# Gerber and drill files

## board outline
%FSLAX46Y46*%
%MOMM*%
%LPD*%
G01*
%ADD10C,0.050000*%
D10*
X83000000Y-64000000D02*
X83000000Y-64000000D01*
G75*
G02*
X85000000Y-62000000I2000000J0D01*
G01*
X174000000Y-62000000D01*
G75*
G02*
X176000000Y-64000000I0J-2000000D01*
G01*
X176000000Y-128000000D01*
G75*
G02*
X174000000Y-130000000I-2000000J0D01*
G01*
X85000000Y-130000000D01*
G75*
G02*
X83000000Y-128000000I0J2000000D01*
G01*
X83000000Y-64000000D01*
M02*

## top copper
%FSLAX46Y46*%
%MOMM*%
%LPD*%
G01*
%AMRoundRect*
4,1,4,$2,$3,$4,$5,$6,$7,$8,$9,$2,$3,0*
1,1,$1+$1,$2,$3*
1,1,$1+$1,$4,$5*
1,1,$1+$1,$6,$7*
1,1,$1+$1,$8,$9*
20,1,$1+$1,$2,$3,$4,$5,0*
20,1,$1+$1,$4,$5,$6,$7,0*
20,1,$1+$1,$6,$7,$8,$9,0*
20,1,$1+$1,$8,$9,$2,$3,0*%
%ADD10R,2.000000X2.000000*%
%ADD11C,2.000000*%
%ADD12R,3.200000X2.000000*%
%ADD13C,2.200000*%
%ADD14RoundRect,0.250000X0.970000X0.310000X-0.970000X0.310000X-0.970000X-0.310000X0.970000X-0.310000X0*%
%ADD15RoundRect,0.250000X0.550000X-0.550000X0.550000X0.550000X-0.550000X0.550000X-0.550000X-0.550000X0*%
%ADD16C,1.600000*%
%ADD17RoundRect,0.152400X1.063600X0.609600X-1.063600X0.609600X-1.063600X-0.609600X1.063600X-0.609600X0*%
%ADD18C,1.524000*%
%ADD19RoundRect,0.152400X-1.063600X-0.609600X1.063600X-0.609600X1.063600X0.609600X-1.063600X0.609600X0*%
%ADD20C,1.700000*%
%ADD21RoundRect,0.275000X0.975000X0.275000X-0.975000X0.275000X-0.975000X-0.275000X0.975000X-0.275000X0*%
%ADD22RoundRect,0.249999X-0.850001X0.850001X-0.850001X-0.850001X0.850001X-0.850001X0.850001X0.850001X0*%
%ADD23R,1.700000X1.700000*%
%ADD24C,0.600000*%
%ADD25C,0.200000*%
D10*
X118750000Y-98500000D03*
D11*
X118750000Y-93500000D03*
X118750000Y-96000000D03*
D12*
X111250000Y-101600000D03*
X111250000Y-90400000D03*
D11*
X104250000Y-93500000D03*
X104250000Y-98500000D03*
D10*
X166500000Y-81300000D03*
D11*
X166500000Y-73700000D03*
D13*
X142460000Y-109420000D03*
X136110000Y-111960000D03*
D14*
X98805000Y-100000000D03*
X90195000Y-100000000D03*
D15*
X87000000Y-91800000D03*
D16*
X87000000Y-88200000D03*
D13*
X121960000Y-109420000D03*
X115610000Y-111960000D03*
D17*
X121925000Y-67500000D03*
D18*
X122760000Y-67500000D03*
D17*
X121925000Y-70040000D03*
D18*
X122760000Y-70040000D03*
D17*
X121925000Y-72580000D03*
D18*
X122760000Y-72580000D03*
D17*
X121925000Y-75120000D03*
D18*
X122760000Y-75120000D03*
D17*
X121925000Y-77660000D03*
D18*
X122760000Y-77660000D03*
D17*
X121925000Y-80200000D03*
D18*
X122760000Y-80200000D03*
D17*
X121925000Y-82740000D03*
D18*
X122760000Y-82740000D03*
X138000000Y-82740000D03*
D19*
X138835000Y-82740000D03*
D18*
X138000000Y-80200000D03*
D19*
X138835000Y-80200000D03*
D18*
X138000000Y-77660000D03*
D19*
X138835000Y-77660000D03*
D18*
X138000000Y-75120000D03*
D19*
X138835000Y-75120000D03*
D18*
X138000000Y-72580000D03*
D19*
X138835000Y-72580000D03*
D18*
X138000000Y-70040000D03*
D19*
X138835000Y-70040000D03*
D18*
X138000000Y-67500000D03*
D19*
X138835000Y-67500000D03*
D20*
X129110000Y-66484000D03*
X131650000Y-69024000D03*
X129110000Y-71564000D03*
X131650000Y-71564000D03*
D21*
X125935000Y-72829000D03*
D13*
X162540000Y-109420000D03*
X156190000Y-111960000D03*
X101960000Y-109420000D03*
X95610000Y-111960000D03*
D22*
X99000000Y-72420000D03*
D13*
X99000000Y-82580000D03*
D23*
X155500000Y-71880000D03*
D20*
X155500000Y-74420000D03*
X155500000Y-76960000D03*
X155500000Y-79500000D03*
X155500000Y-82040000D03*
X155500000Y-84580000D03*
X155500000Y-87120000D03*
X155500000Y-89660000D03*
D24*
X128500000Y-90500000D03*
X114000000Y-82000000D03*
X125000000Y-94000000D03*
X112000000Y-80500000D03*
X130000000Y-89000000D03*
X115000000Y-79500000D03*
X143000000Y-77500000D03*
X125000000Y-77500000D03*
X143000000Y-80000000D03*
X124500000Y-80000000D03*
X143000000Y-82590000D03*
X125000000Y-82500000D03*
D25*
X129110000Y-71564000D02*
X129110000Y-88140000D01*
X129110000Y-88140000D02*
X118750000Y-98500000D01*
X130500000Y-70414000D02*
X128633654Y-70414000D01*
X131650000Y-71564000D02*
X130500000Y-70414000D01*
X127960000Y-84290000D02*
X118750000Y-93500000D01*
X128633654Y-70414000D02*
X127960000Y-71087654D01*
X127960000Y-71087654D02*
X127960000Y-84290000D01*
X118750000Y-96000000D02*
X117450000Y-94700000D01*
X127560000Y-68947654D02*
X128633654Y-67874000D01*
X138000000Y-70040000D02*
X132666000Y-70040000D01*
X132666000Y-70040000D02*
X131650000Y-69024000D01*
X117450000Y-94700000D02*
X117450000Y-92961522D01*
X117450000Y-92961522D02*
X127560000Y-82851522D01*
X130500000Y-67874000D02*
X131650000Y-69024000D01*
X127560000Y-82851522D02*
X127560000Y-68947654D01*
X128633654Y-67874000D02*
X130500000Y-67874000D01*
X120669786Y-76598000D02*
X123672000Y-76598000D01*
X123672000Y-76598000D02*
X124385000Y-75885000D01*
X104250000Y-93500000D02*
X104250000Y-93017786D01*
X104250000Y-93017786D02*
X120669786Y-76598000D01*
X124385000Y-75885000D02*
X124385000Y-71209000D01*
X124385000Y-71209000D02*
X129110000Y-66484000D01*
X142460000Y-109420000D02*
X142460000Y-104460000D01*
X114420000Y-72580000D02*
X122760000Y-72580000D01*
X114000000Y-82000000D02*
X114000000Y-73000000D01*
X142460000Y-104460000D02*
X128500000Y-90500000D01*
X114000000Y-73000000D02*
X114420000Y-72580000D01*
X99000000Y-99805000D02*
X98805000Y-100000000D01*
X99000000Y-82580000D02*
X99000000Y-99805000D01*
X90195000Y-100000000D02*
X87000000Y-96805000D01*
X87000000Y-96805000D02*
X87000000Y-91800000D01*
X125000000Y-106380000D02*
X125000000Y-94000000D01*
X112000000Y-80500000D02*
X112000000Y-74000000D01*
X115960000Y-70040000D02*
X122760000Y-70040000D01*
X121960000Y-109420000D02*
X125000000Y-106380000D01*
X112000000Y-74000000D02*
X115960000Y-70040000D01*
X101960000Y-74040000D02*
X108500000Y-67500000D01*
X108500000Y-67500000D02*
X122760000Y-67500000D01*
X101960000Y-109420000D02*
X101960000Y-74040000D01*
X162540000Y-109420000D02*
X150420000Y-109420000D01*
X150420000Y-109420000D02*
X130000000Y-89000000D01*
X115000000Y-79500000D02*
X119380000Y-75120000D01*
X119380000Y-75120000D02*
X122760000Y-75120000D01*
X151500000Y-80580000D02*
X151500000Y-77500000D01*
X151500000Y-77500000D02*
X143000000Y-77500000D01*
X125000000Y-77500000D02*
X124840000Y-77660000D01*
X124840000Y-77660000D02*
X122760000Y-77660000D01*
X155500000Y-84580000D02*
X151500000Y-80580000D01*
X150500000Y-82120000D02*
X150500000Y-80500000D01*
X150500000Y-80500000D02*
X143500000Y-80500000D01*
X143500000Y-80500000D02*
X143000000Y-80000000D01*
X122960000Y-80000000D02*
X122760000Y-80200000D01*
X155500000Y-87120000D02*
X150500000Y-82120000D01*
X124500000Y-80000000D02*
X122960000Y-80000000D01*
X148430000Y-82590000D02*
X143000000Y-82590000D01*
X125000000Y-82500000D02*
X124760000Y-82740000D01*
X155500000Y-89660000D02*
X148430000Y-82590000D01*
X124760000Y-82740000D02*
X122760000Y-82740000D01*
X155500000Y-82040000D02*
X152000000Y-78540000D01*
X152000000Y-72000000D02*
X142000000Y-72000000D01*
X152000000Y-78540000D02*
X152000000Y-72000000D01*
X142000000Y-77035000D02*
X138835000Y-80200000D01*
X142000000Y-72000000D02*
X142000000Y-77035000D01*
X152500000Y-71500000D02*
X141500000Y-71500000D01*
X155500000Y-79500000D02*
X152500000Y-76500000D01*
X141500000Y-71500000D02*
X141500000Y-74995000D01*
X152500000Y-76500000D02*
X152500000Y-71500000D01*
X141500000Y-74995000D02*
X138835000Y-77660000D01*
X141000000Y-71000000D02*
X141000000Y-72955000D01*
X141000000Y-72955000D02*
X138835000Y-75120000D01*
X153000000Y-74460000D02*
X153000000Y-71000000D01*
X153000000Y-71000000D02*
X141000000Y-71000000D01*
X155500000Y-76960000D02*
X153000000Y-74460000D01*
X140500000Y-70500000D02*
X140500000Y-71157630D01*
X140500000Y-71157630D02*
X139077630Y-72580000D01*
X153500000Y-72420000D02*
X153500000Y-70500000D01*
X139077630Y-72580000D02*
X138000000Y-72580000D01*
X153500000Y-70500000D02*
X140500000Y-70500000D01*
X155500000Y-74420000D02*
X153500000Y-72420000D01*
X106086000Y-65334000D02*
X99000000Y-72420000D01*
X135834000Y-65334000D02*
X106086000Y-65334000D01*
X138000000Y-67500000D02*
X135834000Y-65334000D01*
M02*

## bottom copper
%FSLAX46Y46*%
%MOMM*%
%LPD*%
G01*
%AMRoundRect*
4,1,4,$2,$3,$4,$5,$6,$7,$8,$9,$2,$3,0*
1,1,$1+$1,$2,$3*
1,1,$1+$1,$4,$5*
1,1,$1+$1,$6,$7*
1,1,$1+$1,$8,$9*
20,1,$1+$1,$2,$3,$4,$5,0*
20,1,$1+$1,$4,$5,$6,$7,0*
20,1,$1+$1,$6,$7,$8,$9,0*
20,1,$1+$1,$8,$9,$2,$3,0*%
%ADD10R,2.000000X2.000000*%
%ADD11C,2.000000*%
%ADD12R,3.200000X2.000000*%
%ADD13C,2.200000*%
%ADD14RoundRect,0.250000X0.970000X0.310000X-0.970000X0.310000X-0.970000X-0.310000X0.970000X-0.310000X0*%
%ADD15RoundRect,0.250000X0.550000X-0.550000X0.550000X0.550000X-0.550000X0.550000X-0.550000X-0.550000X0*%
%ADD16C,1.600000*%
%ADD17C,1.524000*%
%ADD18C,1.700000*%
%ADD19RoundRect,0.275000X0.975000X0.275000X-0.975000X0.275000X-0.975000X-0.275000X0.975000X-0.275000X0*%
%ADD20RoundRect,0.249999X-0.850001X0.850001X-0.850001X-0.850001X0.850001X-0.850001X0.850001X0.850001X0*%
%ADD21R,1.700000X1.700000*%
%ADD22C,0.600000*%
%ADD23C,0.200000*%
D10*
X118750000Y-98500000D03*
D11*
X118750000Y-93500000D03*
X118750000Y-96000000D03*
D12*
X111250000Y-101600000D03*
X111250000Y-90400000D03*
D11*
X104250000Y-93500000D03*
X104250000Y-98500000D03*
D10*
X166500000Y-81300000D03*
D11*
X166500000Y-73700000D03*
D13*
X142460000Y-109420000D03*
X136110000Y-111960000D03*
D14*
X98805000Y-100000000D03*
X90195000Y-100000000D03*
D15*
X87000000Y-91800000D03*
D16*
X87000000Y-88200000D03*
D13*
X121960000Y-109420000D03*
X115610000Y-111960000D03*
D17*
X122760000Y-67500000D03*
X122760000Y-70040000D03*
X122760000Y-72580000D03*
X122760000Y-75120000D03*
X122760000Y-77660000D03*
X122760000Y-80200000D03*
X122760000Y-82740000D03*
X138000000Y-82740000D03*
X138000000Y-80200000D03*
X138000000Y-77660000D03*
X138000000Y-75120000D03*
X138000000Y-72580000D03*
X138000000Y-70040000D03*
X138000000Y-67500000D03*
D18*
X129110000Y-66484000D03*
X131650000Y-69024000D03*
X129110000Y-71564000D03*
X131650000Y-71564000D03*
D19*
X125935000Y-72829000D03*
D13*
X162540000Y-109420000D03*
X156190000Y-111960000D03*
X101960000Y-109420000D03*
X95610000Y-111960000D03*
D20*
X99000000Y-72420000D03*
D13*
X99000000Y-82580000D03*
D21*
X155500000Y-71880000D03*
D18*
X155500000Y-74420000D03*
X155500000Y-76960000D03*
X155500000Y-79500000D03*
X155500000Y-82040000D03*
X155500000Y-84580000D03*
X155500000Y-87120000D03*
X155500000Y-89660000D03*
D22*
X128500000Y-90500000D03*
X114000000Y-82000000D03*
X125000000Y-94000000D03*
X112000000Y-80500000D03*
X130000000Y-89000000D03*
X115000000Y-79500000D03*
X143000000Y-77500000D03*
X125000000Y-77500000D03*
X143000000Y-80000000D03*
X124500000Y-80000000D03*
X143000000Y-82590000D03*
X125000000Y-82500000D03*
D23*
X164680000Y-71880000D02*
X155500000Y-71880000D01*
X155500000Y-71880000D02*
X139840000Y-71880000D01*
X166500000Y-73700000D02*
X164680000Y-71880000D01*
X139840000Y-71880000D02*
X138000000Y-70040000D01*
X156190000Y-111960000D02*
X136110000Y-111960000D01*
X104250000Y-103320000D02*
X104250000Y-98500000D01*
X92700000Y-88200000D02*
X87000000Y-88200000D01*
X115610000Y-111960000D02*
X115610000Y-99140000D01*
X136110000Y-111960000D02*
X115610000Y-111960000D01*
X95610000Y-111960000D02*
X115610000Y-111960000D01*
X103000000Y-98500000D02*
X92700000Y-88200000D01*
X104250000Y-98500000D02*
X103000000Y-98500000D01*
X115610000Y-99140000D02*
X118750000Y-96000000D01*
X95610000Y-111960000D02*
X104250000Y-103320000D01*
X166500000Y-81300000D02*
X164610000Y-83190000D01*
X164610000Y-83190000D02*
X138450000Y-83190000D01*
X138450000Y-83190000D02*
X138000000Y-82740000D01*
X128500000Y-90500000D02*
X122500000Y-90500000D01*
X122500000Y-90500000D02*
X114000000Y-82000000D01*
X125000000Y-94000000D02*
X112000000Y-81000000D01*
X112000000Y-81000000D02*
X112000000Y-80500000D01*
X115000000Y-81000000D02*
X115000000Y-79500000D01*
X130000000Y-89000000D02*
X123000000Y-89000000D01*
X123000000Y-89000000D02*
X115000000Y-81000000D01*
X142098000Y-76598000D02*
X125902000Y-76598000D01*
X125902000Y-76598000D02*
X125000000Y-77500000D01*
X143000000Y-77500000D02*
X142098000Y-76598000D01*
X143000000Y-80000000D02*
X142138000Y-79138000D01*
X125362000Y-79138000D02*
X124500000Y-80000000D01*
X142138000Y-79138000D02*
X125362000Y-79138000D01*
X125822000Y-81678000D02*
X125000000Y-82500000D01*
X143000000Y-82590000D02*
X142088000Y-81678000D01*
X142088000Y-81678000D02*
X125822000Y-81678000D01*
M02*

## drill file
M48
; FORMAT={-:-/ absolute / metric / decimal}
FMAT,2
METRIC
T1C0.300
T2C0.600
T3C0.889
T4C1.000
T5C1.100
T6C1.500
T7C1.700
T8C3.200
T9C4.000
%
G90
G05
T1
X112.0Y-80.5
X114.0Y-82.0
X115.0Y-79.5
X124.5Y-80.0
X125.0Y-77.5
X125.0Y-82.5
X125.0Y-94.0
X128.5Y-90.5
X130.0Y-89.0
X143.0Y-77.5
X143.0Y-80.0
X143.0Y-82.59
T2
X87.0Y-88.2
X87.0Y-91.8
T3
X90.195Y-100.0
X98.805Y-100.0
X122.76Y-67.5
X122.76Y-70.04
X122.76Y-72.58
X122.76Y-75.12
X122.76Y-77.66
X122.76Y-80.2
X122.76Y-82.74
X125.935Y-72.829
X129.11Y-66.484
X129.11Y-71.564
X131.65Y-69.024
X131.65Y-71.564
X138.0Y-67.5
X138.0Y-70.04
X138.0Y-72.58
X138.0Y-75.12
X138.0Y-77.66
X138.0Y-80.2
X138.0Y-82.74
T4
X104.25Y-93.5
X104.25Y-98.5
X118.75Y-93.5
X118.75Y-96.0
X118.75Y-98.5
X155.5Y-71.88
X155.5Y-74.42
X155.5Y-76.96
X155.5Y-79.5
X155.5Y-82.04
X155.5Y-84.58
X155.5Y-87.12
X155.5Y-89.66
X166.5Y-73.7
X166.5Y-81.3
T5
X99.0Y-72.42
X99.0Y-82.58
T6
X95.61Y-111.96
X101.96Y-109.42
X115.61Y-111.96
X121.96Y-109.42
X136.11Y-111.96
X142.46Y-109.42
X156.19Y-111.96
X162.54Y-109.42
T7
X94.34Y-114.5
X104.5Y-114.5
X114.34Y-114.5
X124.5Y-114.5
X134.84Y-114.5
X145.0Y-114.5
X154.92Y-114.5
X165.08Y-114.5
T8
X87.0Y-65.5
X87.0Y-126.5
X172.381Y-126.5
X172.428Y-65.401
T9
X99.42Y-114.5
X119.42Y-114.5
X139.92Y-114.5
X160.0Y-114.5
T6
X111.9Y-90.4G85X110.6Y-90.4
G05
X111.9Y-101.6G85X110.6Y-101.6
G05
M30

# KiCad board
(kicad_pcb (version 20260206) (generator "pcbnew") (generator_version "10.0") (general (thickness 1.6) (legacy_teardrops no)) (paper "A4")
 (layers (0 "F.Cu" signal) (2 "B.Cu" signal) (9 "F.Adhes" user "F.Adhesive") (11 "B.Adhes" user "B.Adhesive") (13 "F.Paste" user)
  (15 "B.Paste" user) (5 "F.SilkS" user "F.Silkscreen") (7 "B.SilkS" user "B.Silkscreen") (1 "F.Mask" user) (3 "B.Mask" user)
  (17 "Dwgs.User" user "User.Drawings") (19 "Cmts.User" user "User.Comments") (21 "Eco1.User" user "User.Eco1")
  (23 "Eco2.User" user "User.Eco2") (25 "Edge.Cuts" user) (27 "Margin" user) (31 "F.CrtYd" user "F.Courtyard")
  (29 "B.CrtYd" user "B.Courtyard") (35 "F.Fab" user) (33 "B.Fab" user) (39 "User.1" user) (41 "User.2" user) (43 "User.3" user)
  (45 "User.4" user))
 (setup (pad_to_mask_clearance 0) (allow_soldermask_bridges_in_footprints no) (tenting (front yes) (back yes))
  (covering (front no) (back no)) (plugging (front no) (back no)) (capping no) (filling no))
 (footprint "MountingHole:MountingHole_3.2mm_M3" (layer "F.Cu") (at 172.380609 126.5)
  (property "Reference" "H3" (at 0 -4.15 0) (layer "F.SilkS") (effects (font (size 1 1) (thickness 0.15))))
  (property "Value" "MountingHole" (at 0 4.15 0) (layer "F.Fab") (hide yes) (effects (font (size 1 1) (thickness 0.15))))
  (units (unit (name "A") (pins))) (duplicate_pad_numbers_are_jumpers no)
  (pad "" np_thru_hole circle (at 0 0) (size 3.2 3.2) (drill 3.2) (layers "*.Cu" "*.Mask")))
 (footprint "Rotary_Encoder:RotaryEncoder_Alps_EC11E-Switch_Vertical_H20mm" (layer "F.Cu") (at 118.75 98.5 180)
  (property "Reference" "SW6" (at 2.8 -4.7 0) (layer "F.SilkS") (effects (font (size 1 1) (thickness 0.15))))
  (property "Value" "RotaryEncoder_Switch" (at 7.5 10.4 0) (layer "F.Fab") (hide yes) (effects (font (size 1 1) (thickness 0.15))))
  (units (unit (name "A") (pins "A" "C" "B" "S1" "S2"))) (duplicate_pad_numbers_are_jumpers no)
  (pad "A" thru_hole rect (at 0 0 180) (size 2 2) (drill 1) (layers "*.Cu" "*.Mask") (remove_unused_layers no)
   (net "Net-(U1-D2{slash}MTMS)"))
  (pad "B" thru_hole circle (at 0 5 180) (size 2 2) (drill 1) (layers "*.Cu" "*.Mask") (remove_unused_layers no)
   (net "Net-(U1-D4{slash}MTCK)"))
  (pad "C" thru_hole circle (at 0 2.5 180) (size 2 2) (drill 1) (layers "*.Cu" "*.Mask") (remove_unused_layers no) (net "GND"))
  (pad "MP" thru_hole rect (at 7.5 -3.1 180) (size 3.2 2) (drill oval 2.8 1.5) (layers "*.Cu" "*.Mask") (remove_unused_layers no))
  (pad "MP" thru_hole rect (at 7.5 8.1 180) (size 3.2 2) (drill oval 2.8 1.5) (layers "*.Cu" "*.Mask") (remove_unused_layers no))
  (pad "S1" thru_hole circle (at 14.5 5 180) (size 2 2) (drill 1) (layers "*.Cu" "*.Mask") (remove_unused_layers no)
   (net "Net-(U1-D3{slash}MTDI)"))
  (pad "S2" thru_hole circle (at 14.5 0 180) (size 2 2) (drill 1) (layers "*.Cu" "*.Mask") (remove_unused_layers no) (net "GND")))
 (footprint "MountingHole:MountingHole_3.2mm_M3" (layer "F.Cu") (at 172.4285 65.401372)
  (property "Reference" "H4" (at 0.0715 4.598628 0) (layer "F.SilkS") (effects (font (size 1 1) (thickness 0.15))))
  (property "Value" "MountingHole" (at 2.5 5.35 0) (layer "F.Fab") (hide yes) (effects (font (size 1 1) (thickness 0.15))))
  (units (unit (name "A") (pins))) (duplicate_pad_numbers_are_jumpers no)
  (pad "" np_thru_hole circle (at 0 0) (size 3.2 3.2) (drill 3.2) (layers "*.Cu" "*.Mask")))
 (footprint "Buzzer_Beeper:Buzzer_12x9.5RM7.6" (layer "F.Cu") (at 166.5 81.3 90)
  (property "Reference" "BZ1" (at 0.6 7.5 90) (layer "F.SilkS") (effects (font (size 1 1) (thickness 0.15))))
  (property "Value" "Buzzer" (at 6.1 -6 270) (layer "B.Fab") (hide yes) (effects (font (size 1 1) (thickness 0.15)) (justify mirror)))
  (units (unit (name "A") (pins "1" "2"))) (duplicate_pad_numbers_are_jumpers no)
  (pad "1" thru_hole rect (at 0 0 90) (size 2 2) (drill 1) (layers "*.Cu" "*.Mask") (remove_unused_layers no) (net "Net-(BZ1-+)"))
  (pad "2" thru_hole circle (at 7.6 0 90) (size 2 2) (drill 1) (layers "*.Cu" "*.Mask") (remove_unused_layers no) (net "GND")))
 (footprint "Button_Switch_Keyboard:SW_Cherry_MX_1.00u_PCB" (layer "F.Cu") (at 142.46 109.42)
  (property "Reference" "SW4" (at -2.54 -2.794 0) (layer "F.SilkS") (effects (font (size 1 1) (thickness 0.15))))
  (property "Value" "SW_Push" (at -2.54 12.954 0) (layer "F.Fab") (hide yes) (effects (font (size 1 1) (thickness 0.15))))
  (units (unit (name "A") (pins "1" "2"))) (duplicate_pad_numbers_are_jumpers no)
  (pad "" np_thru_hole circle (at -7.62 5.08) (size 1.7 1.7) (drill 1.7) (layers "*.Cu" "*.Mask"))
  (pad "" np_thru_hole circle (at -2.54 5.08) (size 4 4) (drill 4) (layers "*.Cu" "*.Mask"))
  (pad "" np_thru_hole circle (at 2.54 5.08) (size 1.7 1.7) (drill 1.7) (layers "*.Cu" "*.Mask"))
  (pad "1" thru_hole circle (at 0 0) (size 2.2 2.2) (drill 1.5) (layers "*.Cu" "*.Mask") (remove_unused_layers no) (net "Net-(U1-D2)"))
  (pad "2" thru_hole circle (at -6.35 2.54) (size 2.2 2.2) (drill 1.5) (layers "*.Cu" "*.Mask") (remove_unused_layers no) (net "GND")))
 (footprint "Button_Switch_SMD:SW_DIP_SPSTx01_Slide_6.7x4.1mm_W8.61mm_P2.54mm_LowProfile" (layer "F.Cu") (at 94.5 100 180)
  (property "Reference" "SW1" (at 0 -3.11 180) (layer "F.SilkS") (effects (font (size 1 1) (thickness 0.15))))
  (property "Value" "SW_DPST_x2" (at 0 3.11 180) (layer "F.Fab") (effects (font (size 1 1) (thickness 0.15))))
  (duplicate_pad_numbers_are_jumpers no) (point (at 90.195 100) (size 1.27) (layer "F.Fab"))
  (pad "1" thru_hole roundrect (at -4.305 0 180) (size 2.44 1.12) (drill 0.889) (layers "*.Cu" "*.Mask" "F.Paste") (remove_unused_layers no)
   (roundrect_rratio 0.223214) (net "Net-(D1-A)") (zone_connect 2))
  (pad "2" thru_hole roundrect (at 4.305 0 180) (size 2.44 1.12) (drill 0.889) (layers "*.Cu" "*.Mask") (remove_unused_layers no)
   (roundrect_rratio 0.223214) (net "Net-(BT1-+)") (zone_connect 2)))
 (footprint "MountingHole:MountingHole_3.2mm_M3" (layer "F.Cu") (at 87 126.5)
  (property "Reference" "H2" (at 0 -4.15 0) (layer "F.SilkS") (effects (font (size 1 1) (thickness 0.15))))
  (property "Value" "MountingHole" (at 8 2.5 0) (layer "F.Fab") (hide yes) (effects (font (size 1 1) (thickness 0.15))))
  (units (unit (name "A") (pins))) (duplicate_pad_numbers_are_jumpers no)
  (pad "" np_thru_hole circle (at 0 0) (size 3.2 3.2) (drill 3.2) (layers "*.Cu" "*.Mask")))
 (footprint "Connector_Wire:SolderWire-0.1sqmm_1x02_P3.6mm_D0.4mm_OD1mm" (layer "F.Cu") (at 87 91.8 90)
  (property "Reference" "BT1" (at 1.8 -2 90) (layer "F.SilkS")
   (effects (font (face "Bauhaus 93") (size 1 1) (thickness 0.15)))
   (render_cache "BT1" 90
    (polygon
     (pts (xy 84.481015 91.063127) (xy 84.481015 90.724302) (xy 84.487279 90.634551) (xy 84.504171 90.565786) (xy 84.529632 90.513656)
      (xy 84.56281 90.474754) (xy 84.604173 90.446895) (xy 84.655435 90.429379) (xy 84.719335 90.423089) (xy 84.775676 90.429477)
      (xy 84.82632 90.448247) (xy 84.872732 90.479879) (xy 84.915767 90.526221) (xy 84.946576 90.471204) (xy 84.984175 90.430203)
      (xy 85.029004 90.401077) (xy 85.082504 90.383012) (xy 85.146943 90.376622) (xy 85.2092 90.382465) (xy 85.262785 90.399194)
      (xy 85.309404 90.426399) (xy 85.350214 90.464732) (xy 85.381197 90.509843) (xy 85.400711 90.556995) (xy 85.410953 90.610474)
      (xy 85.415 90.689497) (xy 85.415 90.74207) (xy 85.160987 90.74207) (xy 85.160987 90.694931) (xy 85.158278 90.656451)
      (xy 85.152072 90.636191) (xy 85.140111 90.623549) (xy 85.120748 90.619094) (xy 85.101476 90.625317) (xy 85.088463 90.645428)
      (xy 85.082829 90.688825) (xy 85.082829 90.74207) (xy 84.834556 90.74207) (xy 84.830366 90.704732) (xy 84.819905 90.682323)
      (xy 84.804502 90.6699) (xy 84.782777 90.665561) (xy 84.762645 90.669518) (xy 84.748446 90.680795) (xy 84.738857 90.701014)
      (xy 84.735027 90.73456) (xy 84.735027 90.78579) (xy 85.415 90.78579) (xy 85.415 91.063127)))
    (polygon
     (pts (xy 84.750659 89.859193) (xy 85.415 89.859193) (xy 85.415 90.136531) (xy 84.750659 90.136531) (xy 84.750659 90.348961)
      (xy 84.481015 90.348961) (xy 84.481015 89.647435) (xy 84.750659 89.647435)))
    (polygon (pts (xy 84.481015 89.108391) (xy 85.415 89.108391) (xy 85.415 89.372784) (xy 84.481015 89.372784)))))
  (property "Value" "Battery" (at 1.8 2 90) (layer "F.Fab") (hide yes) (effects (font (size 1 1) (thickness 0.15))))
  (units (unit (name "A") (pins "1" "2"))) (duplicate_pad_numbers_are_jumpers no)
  (pad "1" thru_hole roundrect (at 0 0 90) (size 1.6 1.6) (drill 0.6) (layers "*.Cu" "*.Mask") (remove_unused_layers no)
   (roundrect_rratio 0.15625) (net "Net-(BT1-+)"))
  (pad "2" thru_hole circle (at 3.6 0 90) (size 1.6 1.6) (drill 0.6) (layers "*.Cu" "*.Mask") (remove_unused_layers no) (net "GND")))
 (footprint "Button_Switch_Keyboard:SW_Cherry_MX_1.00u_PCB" (layer "F.Cu") (at 121.96 109.42)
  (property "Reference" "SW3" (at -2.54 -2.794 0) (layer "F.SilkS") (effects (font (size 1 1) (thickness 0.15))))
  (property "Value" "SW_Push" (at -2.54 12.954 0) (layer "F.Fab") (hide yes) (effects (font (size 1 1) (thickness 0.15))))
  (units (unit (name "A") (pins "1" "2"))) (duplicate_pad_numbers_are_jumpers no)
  (pad "" np_thru_hole circle (at -7.62 5.08) (size 1.7 1.7) (drill 1.7) (layers "*.Cu" "*.Mask"))
  (pad "" np_thru_hole circle (at -2.54 5.08) (size 4 4) (drill 4) (layers "*.Cu" "*.Mask"))
  (pad "" np_thru_hole circle (at 2.54 5.08) (size 1.7 1.7) (drill 1.7) (layers "*.Cu" "*.Mask"))
  (pad "1" thru_hole circle (at 0 0) (size 2.2 2.2) (drill 1.5) (layers "*.Cu" "*.Mask") (remove_unused_layers no) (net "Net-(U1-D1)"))
  (pad "2" thru_hole circle (at -6.35 2.54) (size 2.2 2.2) (drill 1.5) (layers "*.Cu" "*.Mask") (remove_unused_layers no) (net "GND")))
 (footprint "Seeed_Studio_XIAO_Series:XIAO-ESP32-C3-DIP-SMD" (layer "F.Cu") (at 130.38 75.12 90)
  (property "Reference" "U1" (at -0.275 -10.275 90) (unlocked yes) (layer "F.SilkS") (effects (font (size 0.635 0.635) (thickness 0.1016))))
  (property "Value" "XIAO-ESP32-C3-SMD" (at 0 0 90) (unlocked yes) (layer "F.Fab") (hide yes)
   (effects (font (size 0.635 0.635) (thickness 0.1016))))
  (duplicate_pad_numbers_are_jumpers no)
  (pad "1" smd roundrect (at 7.62 -8.455 180) (size 2.432 1.524) (layers "F.Cu" "F.Mask") (roundrect_rratio 0.1) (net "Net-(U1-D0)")
   (thermal_bridge_angle 45))
  (pad "1" thru_hole circle (at 7.62 -7.62 180) (size 1.524 1.524) (drill 0.889) (layers "*.Cu" "*.Mask") (remove_unused_layers no)
   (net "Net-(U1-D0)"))
  (pad "2" smd roundrect (at 5.08 -8.455 180) (size 2.432 1.524) (layers "F.Cu" "F.Mask") (roundrect_rratio 0.1) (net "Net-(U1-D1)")
   (thermal_bridge_angle 45))
  (pad "2" thru_hole circle (at 5.08 -7.62 180) (size 1.524 1.524) (drill 0.889) (layers "*.Cu" "*.Mask") (remove_unused_layers no)
   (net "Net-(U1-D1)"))
  (pad "3" smd roundrect (at 2.54 -8.455 180) (size 2.432 1.524) (layers "F.Cu" "F.Mask") (roundrect_rratio 0.1) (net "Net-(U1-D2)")
   (thermal_bridge_angle 45))
  (pad "3" thru_hole circle (at 2.54 -7.62 180) (size 1.524 1.524) (drill 0.889) (layers "*.Cu" "*.Mask") (remove_unused_layers no)
   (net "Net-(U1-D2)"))
  (pad "4" smd roundrect (at 0 -8.455 180) (size 2.432 1.524) (layers "F.Cu" "F.Mask") (roundrect_rratio 0.1) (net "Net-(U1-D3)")
   (thermal_bridge_angle 45))
  (pad "4" thru_hole circle (at 0 -7.62 180) (size 1.524 1.524) (drill 0.889) (layers "*.Cu" "*.Mask") (remove_unused_layers no)
   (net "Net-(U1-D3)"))
  (pad "5" smd roundrect (at -2.54 -8.455 180) (size 2.432 1.524) (layers "F.Cu" "F.Mask") (roundrect_rratio 0.1) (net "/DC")
   (thermal_bridge_angle 45))
  (pad "5" thru_hole circle (at -2.54 -7.62 180) (size 1.524 1.524) (drill 0.889) (layers "*.Cu" "*.Mask") (remove_unused_layers no)
   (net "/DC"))
  (pad "6" smd roundrect (at -5.08 -8.455 180) (size 2.432 1.524) (layers "F.Cu" "F.Mask") (roundrect_rratio 0.1) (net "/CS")
   (thermal_bridge_angle 45))
  (pad "6" thru_hole circle (at -5.08 -7.62 180) (size 1.524 1.524) (drill 0.889) (layers "*.Cu" "*.Mask") (remove_unused_layers no)
   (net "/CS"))
  (pad "7" smd roundrect (at -7.62 -8.455 180) (size 2.432 1.524) (layers "F.Cu" "F.Mask") (roundrect_rratio 0.1) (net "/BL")
   (thermal_bridge_angle 45))
  (pad "7" thru_hole circle (at -7.62 -7.62 180) (size 1.524 1.524) (drill 0.889) (layers "*.Cu" "*.Mask") (remove_unused_layers no)
   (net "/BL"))
  (pad "8" thru_hole circle (at -7.62 7.62) (size 1.524 1.524) (drill 0.889) (layers "*.Cu" "*.Mask") (remove_unused_layers no)
   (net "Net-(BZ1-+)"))
  (pad "8" smd roundrect (at -7.62 8.455) (size 2.432 1.524) (layers "F.Cu" "F.Mask") (roundrect_rratio 0.1) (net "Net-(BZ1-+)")
   (thermal_bridge_angle 45))
  (pad "9" thru_hole circle (at -5.08 7.62) (size 1.524 1.524) (drill 0.889) (layers "*.Cu" "*.Mask") (remove_unused_layers no) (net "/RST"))
  (pad "9" smd roundrect (at -5.08 8.455) (size 2.432 1.524) (layers "F.Cu" "F.Mask") (roundrect_rratio 0.1) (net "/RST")
   (thermal_bridge_angle 45))
  (pad "10" thru_hole circle (at -2.54 7.62) (size 1.524 1.524) (drill 0.889) (layers "*.Cu" "*.Mask") (remove_unused_layers no)
   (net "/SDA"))
  (pad "10" smd roundrect (at -2.54 8.455) (size 2.432 1.524) (layers "F.Cu" "F.Mask") (roundrect_rratio 0.1) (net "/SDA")
   (thermal_bridge_angle 45))
  (pad "11" thru_hole circle (at 0 7.62) (size 1.524 1.524) (drill 0.889) (layers "*.Cu" "*.Mask") (remove_unused_layers no) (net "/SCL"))
  (pad "11" smd roundrect (at 0 8.455) (size 2.432 1.524) (layers "F.Cu" "F.Mask") (roundrect_rratio 0.1) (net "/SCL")
   (thermal_bridge_angle 45))
  (pad "12" thru_hole circle (at 2.54 7.62) (size 1.524 1.524) (drill 0.889) (layers "*.Cu" "*.Mask") (remove_unused_layers no)
   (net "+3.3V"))
  (pad "12" smd roundrect (at 2.54 8.455) (size 2.432 1.524) (layers "F.Cu" "F.Mask") (roundrect_rratio 0.1) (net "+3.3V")
   (thermal_bridge_angle 45))
  (pad "13" thru_hole circle (at 5.08 7.62) (size 1.524 1.524) (drill 0.889) (layers "*.Cu" "*.Mask") (remove_unused_layers no) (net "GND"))
  (pad "13" smd roundrect (at 5.08 8.455) (size 2.432 1.524) (layers "F.Cu" "F.Mask") (roundrect_rratio 0.1) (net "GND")
   (thermal_bridge_angle 45))
  (pad "14" thru_hole circle (at 7.62 7.62) (size 1.524 1.524) (drill 0.889) (layers "*.Cu" "*.Mask") (remove_unused_layers no)
   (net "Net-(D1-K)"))
  (pad "14" smd roundrect (at 7.62 8.455) (size 2.432 1.524) (layers "F.Cu" "F.Mask") (roundrect_rratio 0.1) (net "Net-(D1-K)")
   (thermal_bridge_angle 45))
  (pad "15" thru_hole circle (at 8.636 -1.27) (size 1.7 1.7) (drill 0.889) (layers "*.Cu" "*.Mask") (remove_unused_layers no)
   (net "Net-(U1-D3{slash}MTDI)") (zone_connect 2))
  (pad "18" thru_hole circle (at 6.096 1.27) (size 1.7 1.7) (drill 0.889) (layers "*.Cu" "*.Mask") (remove_unused_layers no) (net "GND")
   (zone_connect 2))
  (pad "19" thru_hole circle (at 3.556 -1.27) (size 1.7 1.7) (drill 0.889) (layers "*.Cu" "*.Mask") (remove_unused_layers no)
   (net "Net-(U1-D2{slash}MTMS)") (zone_connect 2))
  (pad "20" thru_hole circle (at 3.556 1.27) (size 1.7 1.7) (drill 0.889) (layers "*.Cu" "F.Mask") (remove_unused_layers no)
   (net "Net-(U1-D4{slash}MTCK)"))
  (pad "GND" thru_hole roundrect (at 2.291 -4.445 180) (size 2.5 1.1) (drill 0.889) (layers "*.Cu" "*.Mask") (remove_unused_layers no)
   (roundrect_rratio 0.25) (die_length 2) (thermal_bridge_angle 45)))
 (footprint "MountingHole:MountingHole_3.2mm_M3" (layer "F.Cu") (at 87 65.5)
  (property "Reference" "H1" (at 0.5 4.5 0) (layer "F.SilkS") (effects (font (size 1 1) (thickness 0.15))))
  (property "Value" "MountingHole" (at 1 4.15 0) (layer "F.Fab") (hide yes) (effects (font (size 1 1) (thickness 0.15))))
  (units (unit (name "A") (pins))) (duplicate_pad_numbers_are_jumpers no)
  (pad "" np_thru_hole circle (at 0 0) (size 3.2 3.2) (drill 3.2) (layers "*.Cu" "*.Mask")))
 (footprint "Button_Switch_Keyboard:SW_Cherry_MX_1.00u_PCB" (layer "F.Cu") (at 162.54 109.42)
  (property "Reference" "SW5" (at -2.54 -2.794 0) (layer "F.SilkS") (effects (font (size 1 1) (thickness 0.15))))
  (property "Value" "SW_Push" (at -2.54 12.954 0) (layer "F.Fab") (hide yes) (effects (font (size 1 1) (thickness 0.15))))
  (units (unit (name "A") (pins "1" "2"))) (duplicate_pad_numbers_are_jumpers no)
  (pad "" np_thru_hole circle (at -7.62 5.08) (size 1.7 1.7) (drill 1.7) (layers "*.Cu" "*.Mask"))
  (pad "" np_thru_hole circle (at -2.54 5.08) (size 4 4) (drill 4) (layers "*.Cu" "*.Mask"))
  (pad "" np_thru_hole circle (at 2.54 5.08) (size 1.7 1.7) (drill 1.7) (layers "*.Cu" "*.Mask"))
  (pad "1" thru_hole circle (at 0 0) (size 2.2 2.2) (drill 1.5) (layers "*.Cu" "*.Mask") (remove_unused_layers no) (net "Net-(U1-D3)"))
  (pad "2" thru_hole circle (at -6.35 2.54) (size 2.2 2.2) (drill 1.5) (layers "*.Cu" "*.Mask") (remove_unused_layers no) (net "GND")))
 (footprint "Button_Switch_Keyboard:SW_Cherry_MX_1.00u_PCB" (layer "F.Cu") (at 101.96 109.42)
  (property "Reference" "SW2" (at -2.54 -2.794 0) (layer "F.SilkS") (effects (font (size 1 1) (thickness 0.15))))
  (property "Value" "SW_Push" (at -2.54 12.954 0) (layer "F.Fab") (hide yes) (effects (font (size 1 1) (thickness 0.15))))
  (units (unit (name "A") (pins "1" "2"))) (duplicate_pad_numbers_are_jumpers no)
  (pad "" np_thru_hole circle (at -7.62 5.08) (size 1.7 1.7) (drill 1.7) (layers "*.Cu" "*.Mask"))
  (pad "" np_thru_hole circle (at -2.54 5.08) (size 4 4) (drill 4) (layers "*.Cu" "*.Mask"))
  (pad "" np_thru_hole circle (at 2.54 5.08) (size 1.7 1.7) (drill 1.7) (layers "*.Cu" "*.Mask"))
  (pad "1" thru_hole circle (at 0 0) (size 2.2 2.2) (drill 1.5) (layers "*.Cu" "*.Mask") (remove_unused_layers no) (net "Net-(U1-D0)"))
  (pad "2" thru_hole circle (at -6.35 2.54) (size 2.2 2.2) (drill 1.5) (layers "*.Cu" "*.Mask") (remove_unused_layers no) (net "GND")))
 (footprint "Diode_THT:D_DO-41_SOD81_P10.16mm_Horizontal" (layer "B.Cu") (at 99 72.42 -90)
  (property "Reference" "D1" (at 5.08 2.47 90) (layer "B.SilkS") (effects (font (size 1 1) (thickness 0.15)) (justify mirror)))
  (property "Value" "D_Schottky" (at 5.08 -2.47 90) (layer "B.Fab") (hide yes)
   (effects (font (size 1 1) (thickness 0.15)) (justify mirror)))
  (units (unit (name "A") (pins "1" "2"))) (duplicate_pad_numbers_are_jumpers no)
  (pad "1" thru_hole roundrect (at 0 0 270) (size 2.2 2.2) (drill 1.1) (layers "*.Cu" "*.Mask") (remove_unused_layers no)
   (roundrect_rratio 0.113636) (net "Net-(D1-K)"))
  (pad "2" thru_hole circle (at 10.16 0 270) (size 2.2 2.2) (drill 1.1) (layers "*.Cu" "*.Mask") (remove_unused_layers no)
   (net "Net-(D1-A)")))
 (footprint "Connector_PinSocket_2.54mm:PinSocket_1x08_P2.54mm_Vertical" (layer "B.Cu") (at 155.5 71.88 180)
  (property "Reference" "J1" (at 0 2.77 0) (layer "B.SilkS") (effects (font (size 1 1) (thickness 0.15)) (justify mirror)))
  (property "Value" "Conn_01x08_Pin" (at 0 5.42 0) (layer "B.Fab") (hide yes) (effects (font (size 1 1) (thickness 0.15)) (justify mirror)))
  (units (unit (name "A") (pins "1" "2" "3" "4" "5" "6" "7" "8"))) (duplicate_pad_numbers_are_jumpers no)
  (pad "1" thru_hole rect (at 0 0 180) (size 1.7 1.7) (drill 1) (layers "*.Cu" "*.Mask") (remove_unused_layers no) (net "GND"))
  (pad "2" thru_hole circle (at 0 -2.54 180) (size 1.7 1.7) (drill 1) (layers "*.Cu" "*.Mask") (remove_unused_layers no) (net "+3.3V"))
  (pad "3" thru_hole circle (at 0 -5.08 180) (size 1.7 1.7) (drill 1) (layers "*.Cu" "*.Mask") (remove_unused_layers no) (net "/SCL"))
  (pad "4" thru_hole circle (at 0 -7.62 180) (size 1.7 1.7) (drill 1) (layers "*.Cu" "*.Mask") (remove_unused_layers no) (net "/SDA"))
  (pad "5" thru_hole circle (at 0 -10.16 180) (size 1.7 1.7) (drill 1) (layers "*.Cu" "*.Mask") (remove_unused_layers no) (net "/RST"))
  (pad "6" thru_hole circle (at 0 -12.7 180) (size 1.7 1.7) (drill 1) (layers "*.Cu" "*.Mask") (remove_unused_layers no) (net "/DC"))
  (pad "7" thru_hole circle (at 0 -15.24 180) (size 1.7 1.7) (drill 1) (layers "*.Cu" "*.Mask") (remove_unused_layers no) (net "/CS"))
  (pad "8" thru_hole circle (at 0 -17.78 180) (size 1.7 1.7) (drill 1) (layers "*.Cu" "*.Mask") (remove_unused_layers no) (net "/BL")))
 (gr_rect (start 83 62) (end 176 130) (radius 2) (stroke (width 0.05) (type solid)) (fill no) (layer "Edge.Cuts"))
 (segment (start 129.11 71.564) (end 129.11 88.14) (width 0.2) (layer "F.Cu") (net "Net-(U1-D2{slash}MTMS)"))
 (segment (start 129.11 88.14) (end 118.75 98.5) (width 0.2) (layer "F.Cu") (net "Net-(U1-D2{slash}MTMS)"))
 (segment (start 130.5 70.414) (end 128.633654 70.414) (width 0.2) (layer "F.Cu") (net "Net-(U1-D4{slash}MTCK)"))
 (segment (start 131.65 71.564) (end 130.5 70.414) (width 0.2) (layer "F.Cu") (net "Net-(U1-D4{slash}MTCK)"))
 (segment (start 127.96 84.29) (end 118.75 93.5) (width 0.2) (layer "F.Cu") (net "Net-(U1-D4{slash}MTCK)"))
 (segment (start 128.633654 70.414) (end 127.96 71.087654) (width 0.2) (layer "F.Cu") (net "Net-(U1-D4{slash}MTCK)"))
 (segment (start 127.96 71.087654) (end 127.96 84.29) (width 0.2) (layer "F.Cu") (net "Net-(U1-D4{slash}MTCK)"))
 (segment (start 118.75 96) (end 117.45 94.7) (width 0.2) (layer "F.Cu") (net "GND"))
 (segment (start 127.56 68.947654) (end 128.633654 67.874) (width 0.2) (layer "F.Cu") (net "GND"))
 (segment (start 138 70.04) (end 132.666 70.04) (width 0.2) (layer "F.Cu") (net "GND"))
 (segment (start 132.666 70.04) (end 131.65 69.024) (width 0.2) (layer "F.Cu") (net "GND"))
 (segment (start 117.45 94.7) (end 117.45 92.961522) (width 0.2) (layer "F.Cu") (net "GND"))
 (segment (start 117.45 92.961522) (end 127.56 82.851522) (width 0.2) (layer "F.Cu") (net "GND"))
 (segment (start 130.5 67.874) (end 131.65 69.024) (width 0.2) (layer "F.Cu") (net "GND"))
 (segment (start 127.56 82.851522) (end 127.56 68.947654) (width 0.2) (layer "F.Cu") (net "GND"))
 (segment (start 128.633654 67.874) (end 130.5 67.874) (width 0.2) (layer "F.Cu") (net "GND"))
 (segment (start 164.68 71.88) (end 155.5 71.88) (width 0.2) (layer "B.Cu") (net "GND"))
 (segment (start 155.5 71.88) (end 139.84 71.88) (width 0.2) (layer "B.Cu") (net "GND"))
 (segment (start 166.5 73.7) (end 164.68 71.88) (width 0.2) (layer "B.Cu") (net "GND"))
 (segment (start 139.84 71.88) (end 138 70.04) (width 0.2) (layer "B.Cu") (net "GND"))
 (segment (start 156.19 111.96) (end 136.11 111.96) (width 0.2) (layer "B.Cu") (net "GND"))
 (segment (start 104.25 103.32) (end 104.25 98.5) (width 0.2) (layer "B.Cu") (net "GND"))
 (segment (start 92.7 88.2) (end 87 88.2) (width 0.2) (layer "B.Cu") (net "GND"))
 (segment (start 115.61 111.96) (end 115.61 99.14) (width 0.2) (layer "B.Cu") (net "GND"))
 (segment (start 136.11 111.96) (end 115.61 111.96) (width 0.2) (layer "B.Cu") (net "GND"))
 (segment (start 95.61 111.96) (end 115.61 111.96) (width 0.2) (layer "B.Cu") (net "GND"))
 (segment (start 103 98.5) (end 92.7 88.2) (width 0.2) (layer "B.Cu") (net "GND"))
 (segment (start 104.25 98.5) (end 103 98.5) (width 0.2) (layer "B.Cu") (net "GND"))
 (segment (start 115.61 99.14) (end 118.75 96) (width 0.2) (layer "B.Cu") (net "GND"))
 (segment (start 95.61 111.96) (end 104.25 103.32) (width 0.2) (layer "B.Cu") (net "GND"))
 (segment (start 120.669786 76.598) (end 123.672 76.598) (width 0.2) (layer "F.Cu") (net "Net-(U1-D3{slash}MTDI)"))
 (segment (start 123.672 76.598) (end 124.385 75.885) (width 0.2) (layer "F.Cu") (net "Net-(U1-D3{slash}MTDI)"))
 (segment (start 104.25 93.5) (end 104.25 93.017786) (width 0.2) (layer "F.Cu") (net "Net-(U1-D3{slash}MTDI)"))
 (segment (start 104.25 93.017786) (end 120.669786 76.598) (width 0.2) (layer "F.Cu") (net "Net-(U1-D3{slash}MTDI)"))
 (segment (start 124.385 75.885) (end 124.385 71.209) (width 0.2) (layer "F.Cu") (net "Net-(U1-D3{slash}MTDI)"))
 (segment (start 124.385 71.209) (end 129.11 66.484) (width 0.2) (layer "F.Cu") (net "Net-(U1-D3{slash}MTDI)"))
 (segment (start 166.5 81.3) (end 164.61 83.19) (width 0.2) (layer "B.Cu") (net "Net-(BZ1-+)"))
 (segment (start 164.61 83.19) (end 138.45 83.19) (width 0.2) (layer "B.Cu") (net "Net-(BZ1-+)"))
 (segment (start 138.45 83.19) (end 138 82.74) (width 0.2) (layer "B.Cu") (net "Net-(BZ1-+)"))
 (segment (start 142.46 109.42) (end 142.46 104.46) (width 0.2) (layer "F.Cu") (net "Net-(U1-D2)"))
 (segment (start 114.42 72.58) (end 122.76 72.58) (width 0.2) (layer "F.Cu") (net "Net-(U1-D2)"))
 (segment (start 114 82) (end 114 73) (width 0.2) (layer "F.Cu") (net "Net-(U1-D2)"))
 (segment (start 142.46 104.46) (end 128.5 90.5) (width 0.2) (layer "F.Cu") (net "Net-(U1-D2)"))
 (segment (start 114 73) (end 114.42 72.58) (width 0.2) (layer "F.Cu") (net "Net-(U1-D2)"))
 (via (at 128.5 90.5) (size 0.6) (drill 0.3) (layers "F.Cu" "B.Cu") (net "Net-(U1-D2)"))
 (via (at 114 82) (size 0.6) (drill 0.3) (layers "F.Cu" "B.Cu") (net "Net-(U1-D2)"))
 (segment (start 128.5 90.5) (end 122.5 90.5) (width 0.2) (layer "B.Cu") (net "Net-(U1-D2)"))
 (segment (start 122.5 90.5) (end 114 82) (width 0.2) (layer "B.Cu") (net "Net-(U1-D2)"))
 (segment (start 99 99.805) (end 98.805 100) (width 0.2) (layer "F.Cu") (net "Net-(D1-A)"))
 (segment (start 99 82.58) (end 99 99.805) (width 0.2) (layer "F.Cu") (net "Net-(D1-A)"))
 (segment (start 90.195 100) (end 87 96.805) (width 0.2) (layer "F.Cu") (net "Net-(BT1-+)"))
 (segment (start 87 96.805) (end 87 91.8) (width 0.2) (layer "F.Cu") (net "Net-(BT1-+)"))
 (segment (start 125 106.38) (end 125 94) (width 0.2) (layer "F.Cu") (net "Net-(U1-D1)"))
 (segment (start 112 80.5) (end 112 74) (width 0.2) (layer "F.Cu") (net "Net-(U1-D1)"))
 (segment (start 115.96 70.04) (end 122.76 70.04) (width 0.2) (layer "F.Cu") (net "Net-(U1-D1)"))
 (segment (start 121.96 109.42) (end 125 106.38) (width 0.2) (layer "F.Cu") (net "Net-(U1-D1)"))
 (segment (start 112 74) (end 115.96 70.04) (width 0.2) (layer "F.Cu") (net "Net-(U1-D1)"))
 (via (at 125 94) (size 0.6) (drill 0.3) (layers "F.Cu" "B.Cu") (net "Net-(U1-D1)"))
 (via (at 112 80.5) (size 0.6) (drill 0.3) (layers "F.Cu" "B.Cu") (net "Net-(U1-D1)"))
 (segment (start 125 94) (end 112 81) (width 0.2) (layer "B.Cu") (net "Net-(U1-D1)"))
 (segment (start 112 81) (end 112 80.5) (width 0.2) (layer "B.Cu") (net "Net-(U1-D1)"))
 (segment (start 101.96 74.04) (end 108.5 67.5) (width 0.2) (layer "F.Cu") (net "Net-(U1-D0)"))
 (segment (start 108.5 67.5) (end 122.76 67.5) (width 0.2) (layer "F.Cu") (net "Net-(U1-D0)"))
 (segment (start 101.96 109.42) (end 101.96 74.04) (width 0.2) (layer "F.Cu") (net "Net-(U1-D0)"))
 (segment (start 162.54 109.42) (end 150.42 109.42) (width 0.2) (layer "F.Cu") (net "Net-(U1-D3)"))
 (segment (start 150.42 109.42) (end 130 89) (width 0.2) (layer "F.Cu") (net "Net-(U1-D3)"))
 (segment (start 115 79.5) (end 119.38 75.12) (width 0.2) (layer "F.Cu") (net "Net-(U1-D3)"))
 (segment (start 119.38 75.12) (end 122.76 75.12) (width 0.2) (layer "F.Cu") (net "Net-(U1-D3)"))
 (via (at 130 89) (size 0.6) (drill 0.3) (layers "F.Cu" "B.Cu") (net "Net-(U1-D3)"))
 (via (at 115 79.5) (size 0.6) (drill 0.3) (layers "F.Cu" "B.Cu") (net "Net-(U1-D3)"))
 (segment (start 115 81) (end 115 79.5) (width 0.2) (layer "B.Cu") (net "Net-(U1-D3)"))
 (segment (start 130 89) (end 123 89) (width 0.2) (layer "B.Cu") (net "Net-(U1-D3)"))
 (segment (start 123 89) (end 115 81) (width 0.2) (layer "B.Cu") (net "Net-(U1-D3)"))
 (segment (start 151.5 80.58) (end 151.5 77.5) (width 0.2) (layer "F.Cu") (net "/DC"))
 (segment (start 151.5 77.5) (end 143 77.5) (width 0.2) (layer "F.Cu") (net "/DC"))
 (segment (start 125 77.5) (end 124.84 77.66) (width 0.2) (layer "F.Cu") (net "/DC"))
 (segment (start 124.84 77.66) (end 122.76 77.66) (width 0.2) (layer "F.Cu") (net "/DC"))
 (segment (start 155.5 84.58) (end 151.5 80.58) (width 0.2) (layer "F.Cu") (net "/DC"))
 (via (at 143 77.5) (size 0.6) (drill 0.3) (layers "F.Cu" "B.Cu") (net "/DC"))
 (via (at 125 77.5) (size 0.6) (drill 0.3) (layers "F.Cu" "B.Cu") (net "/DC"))
 (segment (start 142.098 76.598) (end 125.902 76.598) (width 0.2) (layer "B.Cu") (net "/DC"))
 (segment (start 125.902 76.598) (end 125 77.5) (width 0.2) (layer "B.Cu") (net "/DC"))
 (segment (start 143 77.5) (end 142.098 76.598) (width 0.2) (layer "B.Cu") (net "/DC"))
 (segment (start 150.5 82.12) (end 150.5 80.5) (width 0.2) (layer "F.Cu") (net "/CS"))
 (segment (start 150.5 80.5) (end 143.5 80.5) (width 0.2) (layer "F.Cu") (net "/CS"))
 (segment (start 143.5 80.5) (end 143 80) (width 0.2) (layer "F.Cu") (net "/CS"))
 (segment (start 122.96 80) (end 122.76 80.2) (width 0.2) (layer "F.Cu") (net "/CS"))
 (segment (start 155.5 87.12) (end 150.5 82.12) (width 0.2) (layer "F.Cu") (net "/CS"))
 (segment (start 124.5 80) (end 122.96 80) (width 0.2) (layer "F.Cu") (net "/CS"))
 (via (at 143 80) (size 0.6) (drill 0.3) (layers "F.Cu" "B.Cu") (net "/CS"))
 (via (at 124.5 80) (size 0.6) (drill 0.3) (layers "F.Cu" "B.Cu") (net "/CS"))
 (segment (start 143 80) (end 142.138 79.138) (width 0.2) (layer "B.Cu") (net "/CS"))
 (segment (start 125.362 79.138) (end 124.5 80) (width 0.2) (layer "B.Cu") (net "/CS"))
 (segment (start 142.138 79.138) (end 125.362 79.138) (width 0.2) (layer "B.Cu") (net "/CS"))
 (segment (start 148.43 82.59) (end 143 82.59) (width 0.2) (layer "F.Cu") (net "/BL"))
 (segment (start 125 82.5) (end 124.76 82.74) (width 0.2) (layer "F.Cu") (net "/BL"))
 (segment (start 155.5 89.66) (end 148.43 82.59) (width 0.2) (layer "F.Cu") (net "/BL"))
 (segment (start 124.76 82.74) (end 122.76 82.74) (width 0.2) (layer "F.Cu") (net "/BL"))
 (via (at 143 82.59) (size 0.6) (drill 0.3) (layers "F.Cu" "B.Cu") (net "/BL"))
 (via (at 125 82.5) (size 0.6) (drill 0.3) (layers "F.Cu" "B.Cu") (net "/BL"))
 (segment (start 125.822 81.678) (end 125 82.5) (width 0.2) (layer "B.Cu") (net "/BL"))
 (segment (start 143 82.59) (end 142.088 81.678) (width 0.2) (layer "B.Cu") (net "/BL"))
 (segment (start 142.088 81.678) (end 125.822 81.678) (width 0.2) (layer "B.Cu") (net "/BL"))
 (segment (start 155.5 82.04) (end 152 78.54) (width 0.2) (layer "F.Cu") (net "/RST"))
 (segment (start 152 72) (end 142 72) (width 0.2) (layer "F.Cu") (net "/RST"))
 (segment (start 152 78.54) (end 152 72) (width 0.2) (layer "F.Cu") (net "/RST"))
 (segment (start 142 77.035) (end 138.835 80.2) (width 0.2) (layer "F.Cu") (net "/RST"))
 (segment (start 142 72) (end 142 77.035) (width 0.2) (layer "F.Cu") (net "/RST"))
 (segment (start 152.5 71.5) (end 141.5 71.5) (width 0.2) (layer "F.Cu") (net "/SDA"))
 (segment (start 155.5 79.5) (end 152.5 76.5) (width 0.2) (layer "F.Cu") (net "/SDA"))
 (segment (start 141.5 71.5) (end 141.5 74.995) (width 0.2) (layer "F.Cu") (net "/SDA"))
 (segment (start 152.5 76.5) (end 152.5 71.5) (width 0.2) (layer "F.Cu") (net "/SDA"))
 (segment (start 141.5 74.995) (end 138.835 77.66) (width 0.2) (layer "F.Cu") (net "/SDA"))
 (segment (start 141 71) (end 141 72.955) (width 0.2) (layer "F.Cu") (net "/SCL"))
 (segment (start 141 72.955) (end 138.835 75.12) (width 0.2) (layer "F.Cu") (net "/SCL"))
 (segment (start 153 74.46) (end 153 71) (width 0.2) (layer "F.Cu") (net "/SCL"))
 (segment (start 153 71) (end 141 71) (width 0.2) (layer "F.Cu") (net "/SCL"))
 (segment (start 155.5 76.96) (end 153 74.46) (width 0.2) (layer "F.Cu") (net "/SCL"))
 (segment (start 140.5 70.5) (end 140.5 71.15763) (width 0.2) (layer "F.Cu") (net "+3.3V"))
 (segment (start 140.5 71.15763) (end 139.07763 72.58) (width 0.2) (layer "F.Cu") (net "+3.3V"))
 (segment (start 153.5 72.42) (end 153.5 70.5) (width 0.2) (layer "F.Cu") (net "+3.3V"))
 (segment (start 139.07763 72.58) (end 138 72.58) (width 0.2) (layer "F.Cu") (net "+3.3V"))
 (segment (start 153.5 70.5) (end 140.5 70.5) (width 0.2) (layer "F.Cu") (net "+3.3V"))
 (segment (start 155.5 74.42) (end 153.5 72.42) (width 0.2) (layer "F.Cu") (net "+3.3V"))
 (segment (start 106.086 65.334) (end 99 72.42) (width 0.2) (layer "F.Cu") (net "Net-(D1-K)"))
 (segment (start 135.834 65.334) (end 106.086 65.334) (width 0.2) (layer "F.Cu") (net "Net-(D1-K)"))
 (segment (start 138 67.5) (end 135.834 65.334) (width 0.2) (layer "F.Cu") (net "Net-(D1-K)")))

